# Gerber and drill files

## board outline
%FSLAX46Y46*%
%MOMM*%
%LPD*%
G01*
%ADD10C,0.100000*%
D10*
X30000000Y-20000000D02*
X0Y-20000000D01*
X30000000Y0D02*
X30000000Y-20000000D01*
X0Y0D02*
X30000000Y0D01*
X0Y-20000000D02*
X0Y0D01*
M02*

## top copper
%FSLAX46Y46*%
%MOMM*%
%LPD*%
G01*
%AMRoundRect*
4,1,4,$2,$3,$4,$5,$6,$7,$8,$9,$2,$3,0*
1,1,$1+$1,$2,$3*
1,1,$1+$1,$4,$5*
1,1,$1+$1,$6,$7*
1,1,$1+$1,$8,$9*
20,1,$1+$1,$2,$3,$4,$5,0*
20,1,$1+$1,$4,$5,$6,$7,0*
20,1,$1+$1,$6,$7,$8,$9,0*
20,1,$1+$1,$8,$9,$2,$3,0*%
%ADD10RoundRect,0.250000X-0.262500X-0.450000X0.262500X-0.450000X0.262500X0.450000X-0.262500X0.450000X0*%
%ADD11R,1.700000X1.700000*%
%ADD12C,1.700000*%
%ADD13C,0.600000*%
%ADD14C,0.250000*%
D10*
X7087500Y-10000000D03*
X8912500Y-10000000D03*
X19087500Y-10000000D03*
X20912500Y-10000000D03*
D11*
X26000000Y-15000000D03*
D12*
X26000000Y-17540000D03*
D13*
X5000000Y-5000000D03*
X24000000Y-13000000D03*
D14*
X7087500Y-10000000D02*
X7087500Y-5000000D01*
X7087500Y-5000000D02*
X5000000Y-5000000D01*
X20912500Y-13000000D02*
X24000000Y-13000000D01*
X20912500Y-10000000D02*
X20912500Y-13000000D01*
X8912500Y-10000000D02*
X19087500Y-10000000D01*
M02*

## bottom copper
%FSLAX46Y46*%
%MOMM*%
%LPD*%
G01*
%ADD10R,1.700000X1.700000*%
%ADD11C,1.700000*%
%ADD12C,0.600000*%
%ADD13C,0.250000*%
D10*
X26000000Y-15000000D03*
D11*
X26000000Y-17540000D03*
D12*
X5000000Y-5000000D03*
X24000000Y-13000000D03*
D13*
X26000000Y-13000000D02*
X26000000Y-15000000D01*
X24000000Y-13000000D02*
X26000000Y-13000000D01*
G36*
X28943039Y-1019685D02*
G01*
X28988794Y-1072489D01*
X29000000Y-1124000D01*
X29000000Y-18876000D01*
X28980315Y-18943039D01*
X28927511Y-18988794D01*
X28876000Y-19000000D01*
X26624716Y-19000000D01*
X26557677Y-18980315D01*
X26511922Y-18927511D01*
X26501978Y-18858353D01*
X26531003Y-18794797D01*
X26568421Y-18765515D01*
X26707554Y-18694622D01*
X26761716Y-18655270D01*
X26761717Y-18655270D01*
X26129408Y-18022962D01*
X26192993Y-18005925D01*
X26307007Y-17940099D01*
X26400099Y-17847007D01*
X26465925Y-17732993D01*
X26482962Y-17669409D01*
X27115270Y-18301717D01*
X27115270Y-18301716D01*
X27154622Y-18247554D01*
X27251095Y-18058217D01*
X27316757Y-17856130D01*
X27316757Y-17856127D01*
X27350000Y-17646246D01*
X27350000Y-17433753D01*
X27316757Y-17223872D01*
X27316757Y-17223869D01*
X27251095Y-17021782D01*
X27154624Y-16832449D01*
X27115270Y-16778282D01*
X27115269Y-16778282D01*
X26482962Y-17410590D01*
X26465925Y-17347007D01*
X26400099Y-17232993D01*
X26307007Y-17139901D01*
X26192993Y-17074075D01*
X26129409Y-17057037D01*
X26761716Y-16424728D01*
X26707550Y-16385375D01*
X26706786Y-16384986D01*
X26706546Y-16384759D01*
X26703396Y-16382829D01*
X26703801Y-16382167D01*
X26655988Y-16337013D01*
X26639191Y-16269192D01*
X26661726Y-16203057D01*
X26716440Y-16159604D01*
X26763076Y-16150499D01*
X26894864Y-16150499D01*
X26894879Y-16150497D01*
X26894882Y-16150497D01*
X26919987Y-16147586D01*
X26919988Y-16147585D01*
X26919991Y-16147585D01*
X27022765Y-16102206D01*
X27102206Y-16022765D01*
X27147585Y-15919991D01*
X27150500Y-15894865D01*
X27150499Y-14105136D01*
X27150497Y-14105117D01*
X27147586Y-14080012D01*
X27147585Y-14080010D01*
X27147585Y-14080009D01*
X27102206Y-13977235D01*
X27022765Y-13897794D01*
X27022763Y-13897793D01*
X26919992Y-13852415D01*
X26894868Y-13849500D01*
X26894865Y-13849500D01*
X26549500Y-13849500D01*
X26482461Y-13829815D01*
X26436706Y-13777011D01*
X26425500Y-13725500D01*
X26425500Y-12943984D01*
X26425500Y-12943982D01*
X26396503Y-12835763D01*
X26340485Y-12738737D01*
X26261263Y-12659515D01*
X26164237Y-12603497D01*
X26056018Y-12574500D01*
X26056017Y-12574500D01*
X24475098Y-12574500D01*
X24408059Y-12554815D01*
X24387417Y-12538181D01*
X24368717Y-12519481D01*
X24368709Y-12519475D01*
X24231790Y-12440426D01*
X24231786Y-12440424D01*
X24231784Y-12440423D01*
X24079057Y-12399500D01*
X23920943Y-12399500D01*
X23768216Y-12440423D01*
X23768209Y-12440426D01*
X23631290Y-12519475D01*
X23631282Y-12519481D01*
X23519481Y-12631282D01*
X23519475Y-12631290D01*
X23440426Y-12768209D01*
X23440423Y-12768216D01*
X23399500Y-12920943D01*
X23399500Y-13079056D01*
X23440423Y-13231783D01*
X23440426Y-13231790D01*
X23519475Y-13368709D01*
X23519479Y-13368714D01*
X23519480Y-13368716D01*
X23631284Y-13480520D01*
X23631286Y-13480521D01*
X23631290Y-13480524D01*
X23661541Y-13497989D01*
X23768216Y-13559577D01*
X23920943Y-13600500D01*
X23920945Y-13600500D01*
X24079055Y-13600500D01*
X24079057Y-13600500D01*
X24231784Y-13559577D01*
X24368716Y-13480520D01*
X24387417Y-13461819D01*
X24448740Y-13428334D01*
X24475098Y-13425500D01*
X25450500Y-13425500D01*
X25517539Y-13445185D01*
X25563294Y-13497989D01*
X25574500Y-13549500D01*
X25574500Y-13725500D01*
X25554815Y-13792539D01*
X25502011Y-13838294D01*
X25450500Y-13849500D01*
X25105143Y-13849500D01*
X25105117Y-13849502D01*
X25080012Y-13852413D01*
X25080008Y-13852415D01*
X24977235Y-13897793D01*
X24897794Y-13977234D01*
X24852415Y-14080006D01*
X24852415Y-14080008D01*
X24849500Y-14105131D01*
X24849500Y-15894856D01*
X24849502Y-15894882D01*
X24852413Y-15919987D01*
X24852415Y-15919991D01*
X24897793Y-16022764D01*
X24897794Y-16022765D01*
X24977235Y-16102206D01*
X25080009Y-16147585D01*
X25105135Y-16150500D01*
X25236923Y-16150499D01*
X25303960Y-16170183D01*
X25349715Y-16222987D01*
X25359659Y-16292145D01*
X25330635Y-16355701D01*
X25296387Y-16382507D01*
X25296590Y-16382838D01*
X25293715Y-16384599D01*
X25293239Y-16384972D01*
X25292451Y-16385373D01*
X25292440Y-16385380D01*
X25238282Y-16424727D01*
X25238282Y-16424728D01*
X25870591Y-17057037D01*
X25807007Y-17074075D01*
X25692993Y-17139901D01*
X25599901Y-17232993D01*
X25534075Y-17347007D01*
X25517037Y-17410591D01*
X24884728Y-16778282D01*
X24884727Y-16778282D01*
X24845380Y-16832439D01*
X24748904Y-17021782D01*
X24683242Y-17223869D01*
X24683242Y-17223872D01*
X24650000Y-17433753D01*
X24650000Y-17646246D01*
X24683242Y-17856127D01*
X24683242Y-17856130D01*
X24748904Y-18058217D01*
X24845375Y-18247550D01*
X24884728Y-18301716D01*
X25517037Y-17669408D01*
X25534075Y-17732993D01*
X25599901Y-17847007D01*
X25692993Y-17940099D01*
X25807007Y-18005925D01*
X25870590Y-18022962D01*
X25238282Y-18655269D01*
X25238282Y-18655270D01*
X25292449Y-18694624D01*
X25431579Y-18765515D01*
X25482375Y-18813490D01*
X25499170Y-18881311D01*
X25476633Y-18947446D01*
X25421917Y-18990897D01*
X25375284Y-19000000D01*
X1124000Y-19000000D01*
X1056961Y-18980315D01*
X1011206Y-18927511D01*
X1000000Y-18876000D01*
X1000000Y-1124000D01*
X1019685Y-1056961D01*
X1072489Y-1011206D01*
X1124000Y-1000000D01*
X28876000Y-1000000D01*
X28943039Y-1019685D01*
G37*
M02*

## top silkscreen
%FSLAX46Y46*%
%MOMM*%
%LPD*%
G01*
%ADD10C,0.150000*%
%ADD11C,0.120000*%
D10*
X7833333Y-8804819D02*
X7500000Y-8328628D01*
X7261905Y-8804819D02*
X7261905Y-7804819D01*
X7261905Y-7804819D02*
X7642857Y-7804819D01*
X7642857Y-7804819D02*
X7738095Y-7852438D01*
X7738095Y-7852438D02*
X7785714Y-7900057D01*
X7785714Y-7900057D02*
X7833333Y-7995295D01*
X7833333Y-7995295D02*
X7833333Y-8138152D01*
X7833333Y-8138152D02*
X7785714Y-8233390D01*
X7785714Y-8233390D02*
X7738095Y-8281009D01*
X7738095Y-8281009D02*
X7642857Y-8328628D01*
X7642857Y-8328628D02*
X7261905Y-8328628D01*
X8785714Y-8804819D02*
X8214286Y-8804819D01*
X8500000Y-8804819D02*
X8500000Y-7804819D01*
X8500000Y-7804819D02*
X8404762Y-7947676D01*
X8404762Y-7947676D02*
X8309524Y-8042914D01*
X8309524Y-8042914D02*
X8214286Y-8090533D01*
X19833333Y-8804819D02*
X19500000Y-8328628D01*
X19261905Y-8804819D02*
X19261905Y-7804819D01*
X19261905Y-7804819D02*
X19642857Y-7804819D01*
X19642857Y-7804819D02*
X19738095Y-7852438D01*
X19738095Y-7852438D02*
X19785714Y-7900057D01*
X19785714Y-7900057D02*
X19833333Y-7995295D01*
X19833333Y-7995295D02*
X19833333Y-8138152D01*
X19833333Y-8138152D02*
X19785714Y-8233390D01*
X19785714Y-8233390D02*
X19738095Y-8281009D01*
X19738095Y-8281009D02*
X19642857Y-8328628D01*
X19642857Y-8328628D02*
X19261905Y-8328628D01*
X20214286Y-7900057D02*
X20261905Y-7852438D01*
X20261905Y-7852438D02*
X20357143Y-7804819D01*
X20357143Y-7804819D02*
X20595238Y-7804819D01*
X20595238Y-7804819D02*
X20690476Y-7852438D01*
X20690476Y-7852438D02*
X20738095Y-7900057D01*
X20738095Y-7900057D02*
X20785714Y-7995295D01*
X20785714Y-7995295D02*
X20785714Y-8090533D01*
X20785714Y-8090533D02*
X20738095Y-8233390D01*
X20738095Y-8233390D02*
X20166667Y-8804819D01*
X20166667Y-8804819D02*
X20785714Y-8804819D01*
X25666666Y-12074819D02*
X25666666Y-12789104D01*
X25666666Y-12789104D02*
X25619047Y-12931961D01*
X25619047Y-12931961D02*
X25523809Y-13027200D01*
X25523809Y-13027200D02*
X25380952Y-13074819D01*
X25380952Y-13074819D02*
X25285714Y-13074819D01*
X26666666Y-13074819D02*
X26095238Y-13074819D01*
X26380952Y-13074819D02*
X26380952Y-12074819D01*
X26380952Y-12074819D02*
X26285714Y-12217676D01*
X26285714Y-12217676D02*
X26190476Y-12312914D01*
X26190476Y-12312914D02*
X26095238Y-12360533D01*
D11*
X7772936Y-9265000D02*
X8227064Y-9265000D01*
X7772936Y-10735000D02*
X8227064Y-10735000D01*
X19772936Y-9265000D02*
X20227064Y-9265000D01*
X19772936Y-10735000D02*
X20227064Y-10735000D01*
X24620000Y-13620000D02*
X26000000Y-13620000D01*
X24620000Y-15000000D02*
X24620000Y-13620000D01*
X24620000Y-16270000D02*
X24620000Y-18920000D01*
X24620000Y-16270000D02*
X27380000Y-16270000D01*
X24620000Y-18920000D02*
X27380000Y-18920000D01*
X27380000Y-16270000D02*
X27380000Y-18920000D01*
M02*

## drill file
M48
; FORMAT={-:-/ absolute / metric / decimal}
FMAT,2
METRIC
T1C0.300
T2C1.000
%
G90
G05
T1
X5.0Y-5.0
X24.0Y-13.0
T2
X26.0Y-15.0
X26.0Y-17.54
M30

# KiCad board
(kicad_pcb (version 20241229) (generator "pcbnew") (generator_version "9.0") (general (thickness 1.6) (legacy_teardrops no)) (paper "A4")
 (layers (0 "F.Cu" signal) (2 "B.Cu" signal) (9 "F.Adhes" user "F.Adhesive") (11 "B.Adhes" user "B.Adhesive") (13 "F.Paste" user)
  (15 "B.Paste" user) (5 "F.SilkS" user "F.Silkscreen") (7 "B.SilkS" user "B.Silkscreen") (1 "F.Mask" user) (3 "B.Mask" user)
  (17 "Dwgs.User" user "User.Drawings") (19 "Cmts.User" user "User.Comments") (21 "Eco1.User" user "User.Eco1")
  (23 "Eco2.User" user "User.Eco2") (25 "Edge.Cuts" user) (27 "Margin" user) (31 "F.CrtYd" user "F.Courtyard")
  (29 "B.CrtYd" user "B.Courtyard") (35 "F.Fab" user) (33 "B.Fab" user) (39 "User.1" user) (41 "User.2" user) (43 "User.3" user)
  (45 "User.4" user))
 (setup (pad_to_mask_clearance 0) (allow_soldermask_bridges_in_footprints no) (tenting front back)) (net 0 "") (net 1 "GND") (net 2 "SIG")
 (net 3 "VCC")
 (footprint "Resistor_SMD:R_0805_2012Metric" (layer "F.Cu") (at 8 10)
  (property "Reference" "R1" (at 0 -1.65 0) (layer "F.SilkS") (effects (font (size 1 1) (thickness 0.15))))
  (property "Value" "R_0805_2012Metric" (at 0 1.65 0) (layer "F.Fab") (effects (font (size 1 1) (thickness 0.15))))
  (fp_line (start -0.227064 -0.735) (end 0.227064 -0.735) (stroke (width 0.12) (type solid)) (layer "F.SilkS"))
  (fp_line (start -0.227064 0.735) (end 0.227064 0.735) (stroke (width 0.12) (type solid)) (layer "F.SilkS"))
  (pad "1" smd roundrect (at -0.9125 0) (size 1.025 1.4) (layers "F.Cu" "F.Mask" "F.Paste") (roundrect_rratio 0.243902) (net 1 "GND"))
  (pad "2" smd roundrect (at 0.9125 0) (size 1.025 1.4) (layers "F.Cu" "F.Mask" "F.Paste") (roundrect_rratio 0.243902) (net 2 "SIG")))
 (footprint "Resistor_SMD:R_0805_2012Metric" (layer "F.Cu") (at 20 10)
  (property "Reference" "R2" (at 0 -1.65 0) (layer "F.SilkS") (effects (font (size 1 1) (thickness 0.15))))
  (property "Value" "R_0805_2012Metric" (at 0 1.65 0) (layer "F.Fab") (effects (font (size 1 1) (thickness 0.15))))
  (fp_line (start -0.227064 -0.735) (end 0.227064 -0.735) (stroke (width 0.12) (type solid)) (layer "F.SilkS"))
  (fp_line (start -0.227064 0.735) (end 0.227064 0.735) (stroke (width 0.12) (type solid)) (layer "F.SilkS"))
  (pad "1" smd roundrect (at -0.9125 0) (size 1.025 1.4) (layers "F.Cu" "F.Mask" "F.Paste") (roundrect_rratio 0.243902) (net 2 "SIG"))
  (pad "2" smd roundrect (at 0.9125 0) (size 1.025 1.4) (layers "F.Cu" "F.Mask" "F.Paste") (roundrect_rratio 0.243902) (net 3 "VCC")))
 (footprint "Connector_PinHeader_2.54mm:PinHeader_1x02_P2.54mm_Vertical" (layer "F.Cu") (at 26 15)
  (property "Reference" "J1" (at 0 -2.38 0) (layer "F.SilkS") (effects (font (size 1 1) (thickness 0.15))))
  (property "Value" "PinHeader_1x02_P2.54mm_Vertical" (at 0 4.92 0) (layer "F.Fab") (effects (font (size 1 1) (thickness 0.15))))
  (fp_line (start -1.38 -1.38) (end 0 -1.38) (stroke (width 0.12) (type solid)) (layer "F.SilkS"))
  (fp_line (start -1.38 0) (end -1.38 -1.38) (stroke (width 0.12) (type solid)) (layer "F.SilkS"))
  (fp_line (start -1.38 1.27) (end -1.38 3.92) (stroke (width 0.12) (type solid)) (layer "F.SilkS"))
  (fp_line (start -1.38 1.27) (end 1.38 1.27) (stroke (width 0.12) (type solid)) (layer "F.SilkS"))
  (fp_line (start -1.38 3.92) (end 1.38 3.92) (stroke (width 0.12) (type solid)) (layer "F.SilkS"))
  (fp_line (start 1.38 1.27) (end 1.38 3.92) (stroke (width 0.12) (type solid)) (layer "F.SilkS"))
  (pad "1" thru_hole rect (at 0 0) (size 1.7 1.7) (drill 1) (layers "*.Cu" "*.Mask") (remove_unused_layers no) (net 3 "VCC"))
  (pad "2" thru_hole circle (at 0 2.54) (size 1.7 1.7) (drill 1) (layers "*.Cu" "*.Mask") (remove_unused_layers no) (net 1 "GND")))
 (gr_line (start 30 20) (end 0 20) (stroke (width 0.1) (type default)) (layer "Edge.Cuts"))
 (gr_line (start 30 0) (end 30 20) (stroke (width 0.1) (type default)) (layer "Edge.Cuts"))
 (gr_line (start 0 0) (end 30 0) (stroke (width 0.1) (type default)) (layer "Edge.Cuts"))
 (gr_line (start 0 20) (end 0 0) (stroke (width 0.1) (type default)) (layer "Edge.Cuts"))
 (segment (start 7.0875 10) (end 7.0875 5) (width 0.25) (layer "F.Cu") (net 1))
 (segment (start 7.0875 5) (end 5 5) (width 0.25) (layer "F.Cu") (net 1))
 (via (at 5 5) (size 0.6) (drill 0.3) (layers "F.Cu" "B.Cu") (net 1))
 (segment (start 20.9125 13) (end 24 13) (width 0.25) (layer "F.Cu") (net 3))
 (segment (start 20.9125 10) (end 20.9125 13) (width 0.25) (layer "F.Cu") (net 3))
 (via (at 24 13) (size 0.6) (drill 0.3) (layers "F.Cu" "B.Cu") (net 3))
 (segment (start 26 13) (end 26 15) (width 0.25) (layer "B.Cu") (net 3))
 (segment (start 24 13) (end 26 13) (width 0.25) (layer "B.Cu") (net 3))
 (segment (start 8.9125 10) (end 19.0875 10) (width 0.25) (layer "F.Cu") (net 2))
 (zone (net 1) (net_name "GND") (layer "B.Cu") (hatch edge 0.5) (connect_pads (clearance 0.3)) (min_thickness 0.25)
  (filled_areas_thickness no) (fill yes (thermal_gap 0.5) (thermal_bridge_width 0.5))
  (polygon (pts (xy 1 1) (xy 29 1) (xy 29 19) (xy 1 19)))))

